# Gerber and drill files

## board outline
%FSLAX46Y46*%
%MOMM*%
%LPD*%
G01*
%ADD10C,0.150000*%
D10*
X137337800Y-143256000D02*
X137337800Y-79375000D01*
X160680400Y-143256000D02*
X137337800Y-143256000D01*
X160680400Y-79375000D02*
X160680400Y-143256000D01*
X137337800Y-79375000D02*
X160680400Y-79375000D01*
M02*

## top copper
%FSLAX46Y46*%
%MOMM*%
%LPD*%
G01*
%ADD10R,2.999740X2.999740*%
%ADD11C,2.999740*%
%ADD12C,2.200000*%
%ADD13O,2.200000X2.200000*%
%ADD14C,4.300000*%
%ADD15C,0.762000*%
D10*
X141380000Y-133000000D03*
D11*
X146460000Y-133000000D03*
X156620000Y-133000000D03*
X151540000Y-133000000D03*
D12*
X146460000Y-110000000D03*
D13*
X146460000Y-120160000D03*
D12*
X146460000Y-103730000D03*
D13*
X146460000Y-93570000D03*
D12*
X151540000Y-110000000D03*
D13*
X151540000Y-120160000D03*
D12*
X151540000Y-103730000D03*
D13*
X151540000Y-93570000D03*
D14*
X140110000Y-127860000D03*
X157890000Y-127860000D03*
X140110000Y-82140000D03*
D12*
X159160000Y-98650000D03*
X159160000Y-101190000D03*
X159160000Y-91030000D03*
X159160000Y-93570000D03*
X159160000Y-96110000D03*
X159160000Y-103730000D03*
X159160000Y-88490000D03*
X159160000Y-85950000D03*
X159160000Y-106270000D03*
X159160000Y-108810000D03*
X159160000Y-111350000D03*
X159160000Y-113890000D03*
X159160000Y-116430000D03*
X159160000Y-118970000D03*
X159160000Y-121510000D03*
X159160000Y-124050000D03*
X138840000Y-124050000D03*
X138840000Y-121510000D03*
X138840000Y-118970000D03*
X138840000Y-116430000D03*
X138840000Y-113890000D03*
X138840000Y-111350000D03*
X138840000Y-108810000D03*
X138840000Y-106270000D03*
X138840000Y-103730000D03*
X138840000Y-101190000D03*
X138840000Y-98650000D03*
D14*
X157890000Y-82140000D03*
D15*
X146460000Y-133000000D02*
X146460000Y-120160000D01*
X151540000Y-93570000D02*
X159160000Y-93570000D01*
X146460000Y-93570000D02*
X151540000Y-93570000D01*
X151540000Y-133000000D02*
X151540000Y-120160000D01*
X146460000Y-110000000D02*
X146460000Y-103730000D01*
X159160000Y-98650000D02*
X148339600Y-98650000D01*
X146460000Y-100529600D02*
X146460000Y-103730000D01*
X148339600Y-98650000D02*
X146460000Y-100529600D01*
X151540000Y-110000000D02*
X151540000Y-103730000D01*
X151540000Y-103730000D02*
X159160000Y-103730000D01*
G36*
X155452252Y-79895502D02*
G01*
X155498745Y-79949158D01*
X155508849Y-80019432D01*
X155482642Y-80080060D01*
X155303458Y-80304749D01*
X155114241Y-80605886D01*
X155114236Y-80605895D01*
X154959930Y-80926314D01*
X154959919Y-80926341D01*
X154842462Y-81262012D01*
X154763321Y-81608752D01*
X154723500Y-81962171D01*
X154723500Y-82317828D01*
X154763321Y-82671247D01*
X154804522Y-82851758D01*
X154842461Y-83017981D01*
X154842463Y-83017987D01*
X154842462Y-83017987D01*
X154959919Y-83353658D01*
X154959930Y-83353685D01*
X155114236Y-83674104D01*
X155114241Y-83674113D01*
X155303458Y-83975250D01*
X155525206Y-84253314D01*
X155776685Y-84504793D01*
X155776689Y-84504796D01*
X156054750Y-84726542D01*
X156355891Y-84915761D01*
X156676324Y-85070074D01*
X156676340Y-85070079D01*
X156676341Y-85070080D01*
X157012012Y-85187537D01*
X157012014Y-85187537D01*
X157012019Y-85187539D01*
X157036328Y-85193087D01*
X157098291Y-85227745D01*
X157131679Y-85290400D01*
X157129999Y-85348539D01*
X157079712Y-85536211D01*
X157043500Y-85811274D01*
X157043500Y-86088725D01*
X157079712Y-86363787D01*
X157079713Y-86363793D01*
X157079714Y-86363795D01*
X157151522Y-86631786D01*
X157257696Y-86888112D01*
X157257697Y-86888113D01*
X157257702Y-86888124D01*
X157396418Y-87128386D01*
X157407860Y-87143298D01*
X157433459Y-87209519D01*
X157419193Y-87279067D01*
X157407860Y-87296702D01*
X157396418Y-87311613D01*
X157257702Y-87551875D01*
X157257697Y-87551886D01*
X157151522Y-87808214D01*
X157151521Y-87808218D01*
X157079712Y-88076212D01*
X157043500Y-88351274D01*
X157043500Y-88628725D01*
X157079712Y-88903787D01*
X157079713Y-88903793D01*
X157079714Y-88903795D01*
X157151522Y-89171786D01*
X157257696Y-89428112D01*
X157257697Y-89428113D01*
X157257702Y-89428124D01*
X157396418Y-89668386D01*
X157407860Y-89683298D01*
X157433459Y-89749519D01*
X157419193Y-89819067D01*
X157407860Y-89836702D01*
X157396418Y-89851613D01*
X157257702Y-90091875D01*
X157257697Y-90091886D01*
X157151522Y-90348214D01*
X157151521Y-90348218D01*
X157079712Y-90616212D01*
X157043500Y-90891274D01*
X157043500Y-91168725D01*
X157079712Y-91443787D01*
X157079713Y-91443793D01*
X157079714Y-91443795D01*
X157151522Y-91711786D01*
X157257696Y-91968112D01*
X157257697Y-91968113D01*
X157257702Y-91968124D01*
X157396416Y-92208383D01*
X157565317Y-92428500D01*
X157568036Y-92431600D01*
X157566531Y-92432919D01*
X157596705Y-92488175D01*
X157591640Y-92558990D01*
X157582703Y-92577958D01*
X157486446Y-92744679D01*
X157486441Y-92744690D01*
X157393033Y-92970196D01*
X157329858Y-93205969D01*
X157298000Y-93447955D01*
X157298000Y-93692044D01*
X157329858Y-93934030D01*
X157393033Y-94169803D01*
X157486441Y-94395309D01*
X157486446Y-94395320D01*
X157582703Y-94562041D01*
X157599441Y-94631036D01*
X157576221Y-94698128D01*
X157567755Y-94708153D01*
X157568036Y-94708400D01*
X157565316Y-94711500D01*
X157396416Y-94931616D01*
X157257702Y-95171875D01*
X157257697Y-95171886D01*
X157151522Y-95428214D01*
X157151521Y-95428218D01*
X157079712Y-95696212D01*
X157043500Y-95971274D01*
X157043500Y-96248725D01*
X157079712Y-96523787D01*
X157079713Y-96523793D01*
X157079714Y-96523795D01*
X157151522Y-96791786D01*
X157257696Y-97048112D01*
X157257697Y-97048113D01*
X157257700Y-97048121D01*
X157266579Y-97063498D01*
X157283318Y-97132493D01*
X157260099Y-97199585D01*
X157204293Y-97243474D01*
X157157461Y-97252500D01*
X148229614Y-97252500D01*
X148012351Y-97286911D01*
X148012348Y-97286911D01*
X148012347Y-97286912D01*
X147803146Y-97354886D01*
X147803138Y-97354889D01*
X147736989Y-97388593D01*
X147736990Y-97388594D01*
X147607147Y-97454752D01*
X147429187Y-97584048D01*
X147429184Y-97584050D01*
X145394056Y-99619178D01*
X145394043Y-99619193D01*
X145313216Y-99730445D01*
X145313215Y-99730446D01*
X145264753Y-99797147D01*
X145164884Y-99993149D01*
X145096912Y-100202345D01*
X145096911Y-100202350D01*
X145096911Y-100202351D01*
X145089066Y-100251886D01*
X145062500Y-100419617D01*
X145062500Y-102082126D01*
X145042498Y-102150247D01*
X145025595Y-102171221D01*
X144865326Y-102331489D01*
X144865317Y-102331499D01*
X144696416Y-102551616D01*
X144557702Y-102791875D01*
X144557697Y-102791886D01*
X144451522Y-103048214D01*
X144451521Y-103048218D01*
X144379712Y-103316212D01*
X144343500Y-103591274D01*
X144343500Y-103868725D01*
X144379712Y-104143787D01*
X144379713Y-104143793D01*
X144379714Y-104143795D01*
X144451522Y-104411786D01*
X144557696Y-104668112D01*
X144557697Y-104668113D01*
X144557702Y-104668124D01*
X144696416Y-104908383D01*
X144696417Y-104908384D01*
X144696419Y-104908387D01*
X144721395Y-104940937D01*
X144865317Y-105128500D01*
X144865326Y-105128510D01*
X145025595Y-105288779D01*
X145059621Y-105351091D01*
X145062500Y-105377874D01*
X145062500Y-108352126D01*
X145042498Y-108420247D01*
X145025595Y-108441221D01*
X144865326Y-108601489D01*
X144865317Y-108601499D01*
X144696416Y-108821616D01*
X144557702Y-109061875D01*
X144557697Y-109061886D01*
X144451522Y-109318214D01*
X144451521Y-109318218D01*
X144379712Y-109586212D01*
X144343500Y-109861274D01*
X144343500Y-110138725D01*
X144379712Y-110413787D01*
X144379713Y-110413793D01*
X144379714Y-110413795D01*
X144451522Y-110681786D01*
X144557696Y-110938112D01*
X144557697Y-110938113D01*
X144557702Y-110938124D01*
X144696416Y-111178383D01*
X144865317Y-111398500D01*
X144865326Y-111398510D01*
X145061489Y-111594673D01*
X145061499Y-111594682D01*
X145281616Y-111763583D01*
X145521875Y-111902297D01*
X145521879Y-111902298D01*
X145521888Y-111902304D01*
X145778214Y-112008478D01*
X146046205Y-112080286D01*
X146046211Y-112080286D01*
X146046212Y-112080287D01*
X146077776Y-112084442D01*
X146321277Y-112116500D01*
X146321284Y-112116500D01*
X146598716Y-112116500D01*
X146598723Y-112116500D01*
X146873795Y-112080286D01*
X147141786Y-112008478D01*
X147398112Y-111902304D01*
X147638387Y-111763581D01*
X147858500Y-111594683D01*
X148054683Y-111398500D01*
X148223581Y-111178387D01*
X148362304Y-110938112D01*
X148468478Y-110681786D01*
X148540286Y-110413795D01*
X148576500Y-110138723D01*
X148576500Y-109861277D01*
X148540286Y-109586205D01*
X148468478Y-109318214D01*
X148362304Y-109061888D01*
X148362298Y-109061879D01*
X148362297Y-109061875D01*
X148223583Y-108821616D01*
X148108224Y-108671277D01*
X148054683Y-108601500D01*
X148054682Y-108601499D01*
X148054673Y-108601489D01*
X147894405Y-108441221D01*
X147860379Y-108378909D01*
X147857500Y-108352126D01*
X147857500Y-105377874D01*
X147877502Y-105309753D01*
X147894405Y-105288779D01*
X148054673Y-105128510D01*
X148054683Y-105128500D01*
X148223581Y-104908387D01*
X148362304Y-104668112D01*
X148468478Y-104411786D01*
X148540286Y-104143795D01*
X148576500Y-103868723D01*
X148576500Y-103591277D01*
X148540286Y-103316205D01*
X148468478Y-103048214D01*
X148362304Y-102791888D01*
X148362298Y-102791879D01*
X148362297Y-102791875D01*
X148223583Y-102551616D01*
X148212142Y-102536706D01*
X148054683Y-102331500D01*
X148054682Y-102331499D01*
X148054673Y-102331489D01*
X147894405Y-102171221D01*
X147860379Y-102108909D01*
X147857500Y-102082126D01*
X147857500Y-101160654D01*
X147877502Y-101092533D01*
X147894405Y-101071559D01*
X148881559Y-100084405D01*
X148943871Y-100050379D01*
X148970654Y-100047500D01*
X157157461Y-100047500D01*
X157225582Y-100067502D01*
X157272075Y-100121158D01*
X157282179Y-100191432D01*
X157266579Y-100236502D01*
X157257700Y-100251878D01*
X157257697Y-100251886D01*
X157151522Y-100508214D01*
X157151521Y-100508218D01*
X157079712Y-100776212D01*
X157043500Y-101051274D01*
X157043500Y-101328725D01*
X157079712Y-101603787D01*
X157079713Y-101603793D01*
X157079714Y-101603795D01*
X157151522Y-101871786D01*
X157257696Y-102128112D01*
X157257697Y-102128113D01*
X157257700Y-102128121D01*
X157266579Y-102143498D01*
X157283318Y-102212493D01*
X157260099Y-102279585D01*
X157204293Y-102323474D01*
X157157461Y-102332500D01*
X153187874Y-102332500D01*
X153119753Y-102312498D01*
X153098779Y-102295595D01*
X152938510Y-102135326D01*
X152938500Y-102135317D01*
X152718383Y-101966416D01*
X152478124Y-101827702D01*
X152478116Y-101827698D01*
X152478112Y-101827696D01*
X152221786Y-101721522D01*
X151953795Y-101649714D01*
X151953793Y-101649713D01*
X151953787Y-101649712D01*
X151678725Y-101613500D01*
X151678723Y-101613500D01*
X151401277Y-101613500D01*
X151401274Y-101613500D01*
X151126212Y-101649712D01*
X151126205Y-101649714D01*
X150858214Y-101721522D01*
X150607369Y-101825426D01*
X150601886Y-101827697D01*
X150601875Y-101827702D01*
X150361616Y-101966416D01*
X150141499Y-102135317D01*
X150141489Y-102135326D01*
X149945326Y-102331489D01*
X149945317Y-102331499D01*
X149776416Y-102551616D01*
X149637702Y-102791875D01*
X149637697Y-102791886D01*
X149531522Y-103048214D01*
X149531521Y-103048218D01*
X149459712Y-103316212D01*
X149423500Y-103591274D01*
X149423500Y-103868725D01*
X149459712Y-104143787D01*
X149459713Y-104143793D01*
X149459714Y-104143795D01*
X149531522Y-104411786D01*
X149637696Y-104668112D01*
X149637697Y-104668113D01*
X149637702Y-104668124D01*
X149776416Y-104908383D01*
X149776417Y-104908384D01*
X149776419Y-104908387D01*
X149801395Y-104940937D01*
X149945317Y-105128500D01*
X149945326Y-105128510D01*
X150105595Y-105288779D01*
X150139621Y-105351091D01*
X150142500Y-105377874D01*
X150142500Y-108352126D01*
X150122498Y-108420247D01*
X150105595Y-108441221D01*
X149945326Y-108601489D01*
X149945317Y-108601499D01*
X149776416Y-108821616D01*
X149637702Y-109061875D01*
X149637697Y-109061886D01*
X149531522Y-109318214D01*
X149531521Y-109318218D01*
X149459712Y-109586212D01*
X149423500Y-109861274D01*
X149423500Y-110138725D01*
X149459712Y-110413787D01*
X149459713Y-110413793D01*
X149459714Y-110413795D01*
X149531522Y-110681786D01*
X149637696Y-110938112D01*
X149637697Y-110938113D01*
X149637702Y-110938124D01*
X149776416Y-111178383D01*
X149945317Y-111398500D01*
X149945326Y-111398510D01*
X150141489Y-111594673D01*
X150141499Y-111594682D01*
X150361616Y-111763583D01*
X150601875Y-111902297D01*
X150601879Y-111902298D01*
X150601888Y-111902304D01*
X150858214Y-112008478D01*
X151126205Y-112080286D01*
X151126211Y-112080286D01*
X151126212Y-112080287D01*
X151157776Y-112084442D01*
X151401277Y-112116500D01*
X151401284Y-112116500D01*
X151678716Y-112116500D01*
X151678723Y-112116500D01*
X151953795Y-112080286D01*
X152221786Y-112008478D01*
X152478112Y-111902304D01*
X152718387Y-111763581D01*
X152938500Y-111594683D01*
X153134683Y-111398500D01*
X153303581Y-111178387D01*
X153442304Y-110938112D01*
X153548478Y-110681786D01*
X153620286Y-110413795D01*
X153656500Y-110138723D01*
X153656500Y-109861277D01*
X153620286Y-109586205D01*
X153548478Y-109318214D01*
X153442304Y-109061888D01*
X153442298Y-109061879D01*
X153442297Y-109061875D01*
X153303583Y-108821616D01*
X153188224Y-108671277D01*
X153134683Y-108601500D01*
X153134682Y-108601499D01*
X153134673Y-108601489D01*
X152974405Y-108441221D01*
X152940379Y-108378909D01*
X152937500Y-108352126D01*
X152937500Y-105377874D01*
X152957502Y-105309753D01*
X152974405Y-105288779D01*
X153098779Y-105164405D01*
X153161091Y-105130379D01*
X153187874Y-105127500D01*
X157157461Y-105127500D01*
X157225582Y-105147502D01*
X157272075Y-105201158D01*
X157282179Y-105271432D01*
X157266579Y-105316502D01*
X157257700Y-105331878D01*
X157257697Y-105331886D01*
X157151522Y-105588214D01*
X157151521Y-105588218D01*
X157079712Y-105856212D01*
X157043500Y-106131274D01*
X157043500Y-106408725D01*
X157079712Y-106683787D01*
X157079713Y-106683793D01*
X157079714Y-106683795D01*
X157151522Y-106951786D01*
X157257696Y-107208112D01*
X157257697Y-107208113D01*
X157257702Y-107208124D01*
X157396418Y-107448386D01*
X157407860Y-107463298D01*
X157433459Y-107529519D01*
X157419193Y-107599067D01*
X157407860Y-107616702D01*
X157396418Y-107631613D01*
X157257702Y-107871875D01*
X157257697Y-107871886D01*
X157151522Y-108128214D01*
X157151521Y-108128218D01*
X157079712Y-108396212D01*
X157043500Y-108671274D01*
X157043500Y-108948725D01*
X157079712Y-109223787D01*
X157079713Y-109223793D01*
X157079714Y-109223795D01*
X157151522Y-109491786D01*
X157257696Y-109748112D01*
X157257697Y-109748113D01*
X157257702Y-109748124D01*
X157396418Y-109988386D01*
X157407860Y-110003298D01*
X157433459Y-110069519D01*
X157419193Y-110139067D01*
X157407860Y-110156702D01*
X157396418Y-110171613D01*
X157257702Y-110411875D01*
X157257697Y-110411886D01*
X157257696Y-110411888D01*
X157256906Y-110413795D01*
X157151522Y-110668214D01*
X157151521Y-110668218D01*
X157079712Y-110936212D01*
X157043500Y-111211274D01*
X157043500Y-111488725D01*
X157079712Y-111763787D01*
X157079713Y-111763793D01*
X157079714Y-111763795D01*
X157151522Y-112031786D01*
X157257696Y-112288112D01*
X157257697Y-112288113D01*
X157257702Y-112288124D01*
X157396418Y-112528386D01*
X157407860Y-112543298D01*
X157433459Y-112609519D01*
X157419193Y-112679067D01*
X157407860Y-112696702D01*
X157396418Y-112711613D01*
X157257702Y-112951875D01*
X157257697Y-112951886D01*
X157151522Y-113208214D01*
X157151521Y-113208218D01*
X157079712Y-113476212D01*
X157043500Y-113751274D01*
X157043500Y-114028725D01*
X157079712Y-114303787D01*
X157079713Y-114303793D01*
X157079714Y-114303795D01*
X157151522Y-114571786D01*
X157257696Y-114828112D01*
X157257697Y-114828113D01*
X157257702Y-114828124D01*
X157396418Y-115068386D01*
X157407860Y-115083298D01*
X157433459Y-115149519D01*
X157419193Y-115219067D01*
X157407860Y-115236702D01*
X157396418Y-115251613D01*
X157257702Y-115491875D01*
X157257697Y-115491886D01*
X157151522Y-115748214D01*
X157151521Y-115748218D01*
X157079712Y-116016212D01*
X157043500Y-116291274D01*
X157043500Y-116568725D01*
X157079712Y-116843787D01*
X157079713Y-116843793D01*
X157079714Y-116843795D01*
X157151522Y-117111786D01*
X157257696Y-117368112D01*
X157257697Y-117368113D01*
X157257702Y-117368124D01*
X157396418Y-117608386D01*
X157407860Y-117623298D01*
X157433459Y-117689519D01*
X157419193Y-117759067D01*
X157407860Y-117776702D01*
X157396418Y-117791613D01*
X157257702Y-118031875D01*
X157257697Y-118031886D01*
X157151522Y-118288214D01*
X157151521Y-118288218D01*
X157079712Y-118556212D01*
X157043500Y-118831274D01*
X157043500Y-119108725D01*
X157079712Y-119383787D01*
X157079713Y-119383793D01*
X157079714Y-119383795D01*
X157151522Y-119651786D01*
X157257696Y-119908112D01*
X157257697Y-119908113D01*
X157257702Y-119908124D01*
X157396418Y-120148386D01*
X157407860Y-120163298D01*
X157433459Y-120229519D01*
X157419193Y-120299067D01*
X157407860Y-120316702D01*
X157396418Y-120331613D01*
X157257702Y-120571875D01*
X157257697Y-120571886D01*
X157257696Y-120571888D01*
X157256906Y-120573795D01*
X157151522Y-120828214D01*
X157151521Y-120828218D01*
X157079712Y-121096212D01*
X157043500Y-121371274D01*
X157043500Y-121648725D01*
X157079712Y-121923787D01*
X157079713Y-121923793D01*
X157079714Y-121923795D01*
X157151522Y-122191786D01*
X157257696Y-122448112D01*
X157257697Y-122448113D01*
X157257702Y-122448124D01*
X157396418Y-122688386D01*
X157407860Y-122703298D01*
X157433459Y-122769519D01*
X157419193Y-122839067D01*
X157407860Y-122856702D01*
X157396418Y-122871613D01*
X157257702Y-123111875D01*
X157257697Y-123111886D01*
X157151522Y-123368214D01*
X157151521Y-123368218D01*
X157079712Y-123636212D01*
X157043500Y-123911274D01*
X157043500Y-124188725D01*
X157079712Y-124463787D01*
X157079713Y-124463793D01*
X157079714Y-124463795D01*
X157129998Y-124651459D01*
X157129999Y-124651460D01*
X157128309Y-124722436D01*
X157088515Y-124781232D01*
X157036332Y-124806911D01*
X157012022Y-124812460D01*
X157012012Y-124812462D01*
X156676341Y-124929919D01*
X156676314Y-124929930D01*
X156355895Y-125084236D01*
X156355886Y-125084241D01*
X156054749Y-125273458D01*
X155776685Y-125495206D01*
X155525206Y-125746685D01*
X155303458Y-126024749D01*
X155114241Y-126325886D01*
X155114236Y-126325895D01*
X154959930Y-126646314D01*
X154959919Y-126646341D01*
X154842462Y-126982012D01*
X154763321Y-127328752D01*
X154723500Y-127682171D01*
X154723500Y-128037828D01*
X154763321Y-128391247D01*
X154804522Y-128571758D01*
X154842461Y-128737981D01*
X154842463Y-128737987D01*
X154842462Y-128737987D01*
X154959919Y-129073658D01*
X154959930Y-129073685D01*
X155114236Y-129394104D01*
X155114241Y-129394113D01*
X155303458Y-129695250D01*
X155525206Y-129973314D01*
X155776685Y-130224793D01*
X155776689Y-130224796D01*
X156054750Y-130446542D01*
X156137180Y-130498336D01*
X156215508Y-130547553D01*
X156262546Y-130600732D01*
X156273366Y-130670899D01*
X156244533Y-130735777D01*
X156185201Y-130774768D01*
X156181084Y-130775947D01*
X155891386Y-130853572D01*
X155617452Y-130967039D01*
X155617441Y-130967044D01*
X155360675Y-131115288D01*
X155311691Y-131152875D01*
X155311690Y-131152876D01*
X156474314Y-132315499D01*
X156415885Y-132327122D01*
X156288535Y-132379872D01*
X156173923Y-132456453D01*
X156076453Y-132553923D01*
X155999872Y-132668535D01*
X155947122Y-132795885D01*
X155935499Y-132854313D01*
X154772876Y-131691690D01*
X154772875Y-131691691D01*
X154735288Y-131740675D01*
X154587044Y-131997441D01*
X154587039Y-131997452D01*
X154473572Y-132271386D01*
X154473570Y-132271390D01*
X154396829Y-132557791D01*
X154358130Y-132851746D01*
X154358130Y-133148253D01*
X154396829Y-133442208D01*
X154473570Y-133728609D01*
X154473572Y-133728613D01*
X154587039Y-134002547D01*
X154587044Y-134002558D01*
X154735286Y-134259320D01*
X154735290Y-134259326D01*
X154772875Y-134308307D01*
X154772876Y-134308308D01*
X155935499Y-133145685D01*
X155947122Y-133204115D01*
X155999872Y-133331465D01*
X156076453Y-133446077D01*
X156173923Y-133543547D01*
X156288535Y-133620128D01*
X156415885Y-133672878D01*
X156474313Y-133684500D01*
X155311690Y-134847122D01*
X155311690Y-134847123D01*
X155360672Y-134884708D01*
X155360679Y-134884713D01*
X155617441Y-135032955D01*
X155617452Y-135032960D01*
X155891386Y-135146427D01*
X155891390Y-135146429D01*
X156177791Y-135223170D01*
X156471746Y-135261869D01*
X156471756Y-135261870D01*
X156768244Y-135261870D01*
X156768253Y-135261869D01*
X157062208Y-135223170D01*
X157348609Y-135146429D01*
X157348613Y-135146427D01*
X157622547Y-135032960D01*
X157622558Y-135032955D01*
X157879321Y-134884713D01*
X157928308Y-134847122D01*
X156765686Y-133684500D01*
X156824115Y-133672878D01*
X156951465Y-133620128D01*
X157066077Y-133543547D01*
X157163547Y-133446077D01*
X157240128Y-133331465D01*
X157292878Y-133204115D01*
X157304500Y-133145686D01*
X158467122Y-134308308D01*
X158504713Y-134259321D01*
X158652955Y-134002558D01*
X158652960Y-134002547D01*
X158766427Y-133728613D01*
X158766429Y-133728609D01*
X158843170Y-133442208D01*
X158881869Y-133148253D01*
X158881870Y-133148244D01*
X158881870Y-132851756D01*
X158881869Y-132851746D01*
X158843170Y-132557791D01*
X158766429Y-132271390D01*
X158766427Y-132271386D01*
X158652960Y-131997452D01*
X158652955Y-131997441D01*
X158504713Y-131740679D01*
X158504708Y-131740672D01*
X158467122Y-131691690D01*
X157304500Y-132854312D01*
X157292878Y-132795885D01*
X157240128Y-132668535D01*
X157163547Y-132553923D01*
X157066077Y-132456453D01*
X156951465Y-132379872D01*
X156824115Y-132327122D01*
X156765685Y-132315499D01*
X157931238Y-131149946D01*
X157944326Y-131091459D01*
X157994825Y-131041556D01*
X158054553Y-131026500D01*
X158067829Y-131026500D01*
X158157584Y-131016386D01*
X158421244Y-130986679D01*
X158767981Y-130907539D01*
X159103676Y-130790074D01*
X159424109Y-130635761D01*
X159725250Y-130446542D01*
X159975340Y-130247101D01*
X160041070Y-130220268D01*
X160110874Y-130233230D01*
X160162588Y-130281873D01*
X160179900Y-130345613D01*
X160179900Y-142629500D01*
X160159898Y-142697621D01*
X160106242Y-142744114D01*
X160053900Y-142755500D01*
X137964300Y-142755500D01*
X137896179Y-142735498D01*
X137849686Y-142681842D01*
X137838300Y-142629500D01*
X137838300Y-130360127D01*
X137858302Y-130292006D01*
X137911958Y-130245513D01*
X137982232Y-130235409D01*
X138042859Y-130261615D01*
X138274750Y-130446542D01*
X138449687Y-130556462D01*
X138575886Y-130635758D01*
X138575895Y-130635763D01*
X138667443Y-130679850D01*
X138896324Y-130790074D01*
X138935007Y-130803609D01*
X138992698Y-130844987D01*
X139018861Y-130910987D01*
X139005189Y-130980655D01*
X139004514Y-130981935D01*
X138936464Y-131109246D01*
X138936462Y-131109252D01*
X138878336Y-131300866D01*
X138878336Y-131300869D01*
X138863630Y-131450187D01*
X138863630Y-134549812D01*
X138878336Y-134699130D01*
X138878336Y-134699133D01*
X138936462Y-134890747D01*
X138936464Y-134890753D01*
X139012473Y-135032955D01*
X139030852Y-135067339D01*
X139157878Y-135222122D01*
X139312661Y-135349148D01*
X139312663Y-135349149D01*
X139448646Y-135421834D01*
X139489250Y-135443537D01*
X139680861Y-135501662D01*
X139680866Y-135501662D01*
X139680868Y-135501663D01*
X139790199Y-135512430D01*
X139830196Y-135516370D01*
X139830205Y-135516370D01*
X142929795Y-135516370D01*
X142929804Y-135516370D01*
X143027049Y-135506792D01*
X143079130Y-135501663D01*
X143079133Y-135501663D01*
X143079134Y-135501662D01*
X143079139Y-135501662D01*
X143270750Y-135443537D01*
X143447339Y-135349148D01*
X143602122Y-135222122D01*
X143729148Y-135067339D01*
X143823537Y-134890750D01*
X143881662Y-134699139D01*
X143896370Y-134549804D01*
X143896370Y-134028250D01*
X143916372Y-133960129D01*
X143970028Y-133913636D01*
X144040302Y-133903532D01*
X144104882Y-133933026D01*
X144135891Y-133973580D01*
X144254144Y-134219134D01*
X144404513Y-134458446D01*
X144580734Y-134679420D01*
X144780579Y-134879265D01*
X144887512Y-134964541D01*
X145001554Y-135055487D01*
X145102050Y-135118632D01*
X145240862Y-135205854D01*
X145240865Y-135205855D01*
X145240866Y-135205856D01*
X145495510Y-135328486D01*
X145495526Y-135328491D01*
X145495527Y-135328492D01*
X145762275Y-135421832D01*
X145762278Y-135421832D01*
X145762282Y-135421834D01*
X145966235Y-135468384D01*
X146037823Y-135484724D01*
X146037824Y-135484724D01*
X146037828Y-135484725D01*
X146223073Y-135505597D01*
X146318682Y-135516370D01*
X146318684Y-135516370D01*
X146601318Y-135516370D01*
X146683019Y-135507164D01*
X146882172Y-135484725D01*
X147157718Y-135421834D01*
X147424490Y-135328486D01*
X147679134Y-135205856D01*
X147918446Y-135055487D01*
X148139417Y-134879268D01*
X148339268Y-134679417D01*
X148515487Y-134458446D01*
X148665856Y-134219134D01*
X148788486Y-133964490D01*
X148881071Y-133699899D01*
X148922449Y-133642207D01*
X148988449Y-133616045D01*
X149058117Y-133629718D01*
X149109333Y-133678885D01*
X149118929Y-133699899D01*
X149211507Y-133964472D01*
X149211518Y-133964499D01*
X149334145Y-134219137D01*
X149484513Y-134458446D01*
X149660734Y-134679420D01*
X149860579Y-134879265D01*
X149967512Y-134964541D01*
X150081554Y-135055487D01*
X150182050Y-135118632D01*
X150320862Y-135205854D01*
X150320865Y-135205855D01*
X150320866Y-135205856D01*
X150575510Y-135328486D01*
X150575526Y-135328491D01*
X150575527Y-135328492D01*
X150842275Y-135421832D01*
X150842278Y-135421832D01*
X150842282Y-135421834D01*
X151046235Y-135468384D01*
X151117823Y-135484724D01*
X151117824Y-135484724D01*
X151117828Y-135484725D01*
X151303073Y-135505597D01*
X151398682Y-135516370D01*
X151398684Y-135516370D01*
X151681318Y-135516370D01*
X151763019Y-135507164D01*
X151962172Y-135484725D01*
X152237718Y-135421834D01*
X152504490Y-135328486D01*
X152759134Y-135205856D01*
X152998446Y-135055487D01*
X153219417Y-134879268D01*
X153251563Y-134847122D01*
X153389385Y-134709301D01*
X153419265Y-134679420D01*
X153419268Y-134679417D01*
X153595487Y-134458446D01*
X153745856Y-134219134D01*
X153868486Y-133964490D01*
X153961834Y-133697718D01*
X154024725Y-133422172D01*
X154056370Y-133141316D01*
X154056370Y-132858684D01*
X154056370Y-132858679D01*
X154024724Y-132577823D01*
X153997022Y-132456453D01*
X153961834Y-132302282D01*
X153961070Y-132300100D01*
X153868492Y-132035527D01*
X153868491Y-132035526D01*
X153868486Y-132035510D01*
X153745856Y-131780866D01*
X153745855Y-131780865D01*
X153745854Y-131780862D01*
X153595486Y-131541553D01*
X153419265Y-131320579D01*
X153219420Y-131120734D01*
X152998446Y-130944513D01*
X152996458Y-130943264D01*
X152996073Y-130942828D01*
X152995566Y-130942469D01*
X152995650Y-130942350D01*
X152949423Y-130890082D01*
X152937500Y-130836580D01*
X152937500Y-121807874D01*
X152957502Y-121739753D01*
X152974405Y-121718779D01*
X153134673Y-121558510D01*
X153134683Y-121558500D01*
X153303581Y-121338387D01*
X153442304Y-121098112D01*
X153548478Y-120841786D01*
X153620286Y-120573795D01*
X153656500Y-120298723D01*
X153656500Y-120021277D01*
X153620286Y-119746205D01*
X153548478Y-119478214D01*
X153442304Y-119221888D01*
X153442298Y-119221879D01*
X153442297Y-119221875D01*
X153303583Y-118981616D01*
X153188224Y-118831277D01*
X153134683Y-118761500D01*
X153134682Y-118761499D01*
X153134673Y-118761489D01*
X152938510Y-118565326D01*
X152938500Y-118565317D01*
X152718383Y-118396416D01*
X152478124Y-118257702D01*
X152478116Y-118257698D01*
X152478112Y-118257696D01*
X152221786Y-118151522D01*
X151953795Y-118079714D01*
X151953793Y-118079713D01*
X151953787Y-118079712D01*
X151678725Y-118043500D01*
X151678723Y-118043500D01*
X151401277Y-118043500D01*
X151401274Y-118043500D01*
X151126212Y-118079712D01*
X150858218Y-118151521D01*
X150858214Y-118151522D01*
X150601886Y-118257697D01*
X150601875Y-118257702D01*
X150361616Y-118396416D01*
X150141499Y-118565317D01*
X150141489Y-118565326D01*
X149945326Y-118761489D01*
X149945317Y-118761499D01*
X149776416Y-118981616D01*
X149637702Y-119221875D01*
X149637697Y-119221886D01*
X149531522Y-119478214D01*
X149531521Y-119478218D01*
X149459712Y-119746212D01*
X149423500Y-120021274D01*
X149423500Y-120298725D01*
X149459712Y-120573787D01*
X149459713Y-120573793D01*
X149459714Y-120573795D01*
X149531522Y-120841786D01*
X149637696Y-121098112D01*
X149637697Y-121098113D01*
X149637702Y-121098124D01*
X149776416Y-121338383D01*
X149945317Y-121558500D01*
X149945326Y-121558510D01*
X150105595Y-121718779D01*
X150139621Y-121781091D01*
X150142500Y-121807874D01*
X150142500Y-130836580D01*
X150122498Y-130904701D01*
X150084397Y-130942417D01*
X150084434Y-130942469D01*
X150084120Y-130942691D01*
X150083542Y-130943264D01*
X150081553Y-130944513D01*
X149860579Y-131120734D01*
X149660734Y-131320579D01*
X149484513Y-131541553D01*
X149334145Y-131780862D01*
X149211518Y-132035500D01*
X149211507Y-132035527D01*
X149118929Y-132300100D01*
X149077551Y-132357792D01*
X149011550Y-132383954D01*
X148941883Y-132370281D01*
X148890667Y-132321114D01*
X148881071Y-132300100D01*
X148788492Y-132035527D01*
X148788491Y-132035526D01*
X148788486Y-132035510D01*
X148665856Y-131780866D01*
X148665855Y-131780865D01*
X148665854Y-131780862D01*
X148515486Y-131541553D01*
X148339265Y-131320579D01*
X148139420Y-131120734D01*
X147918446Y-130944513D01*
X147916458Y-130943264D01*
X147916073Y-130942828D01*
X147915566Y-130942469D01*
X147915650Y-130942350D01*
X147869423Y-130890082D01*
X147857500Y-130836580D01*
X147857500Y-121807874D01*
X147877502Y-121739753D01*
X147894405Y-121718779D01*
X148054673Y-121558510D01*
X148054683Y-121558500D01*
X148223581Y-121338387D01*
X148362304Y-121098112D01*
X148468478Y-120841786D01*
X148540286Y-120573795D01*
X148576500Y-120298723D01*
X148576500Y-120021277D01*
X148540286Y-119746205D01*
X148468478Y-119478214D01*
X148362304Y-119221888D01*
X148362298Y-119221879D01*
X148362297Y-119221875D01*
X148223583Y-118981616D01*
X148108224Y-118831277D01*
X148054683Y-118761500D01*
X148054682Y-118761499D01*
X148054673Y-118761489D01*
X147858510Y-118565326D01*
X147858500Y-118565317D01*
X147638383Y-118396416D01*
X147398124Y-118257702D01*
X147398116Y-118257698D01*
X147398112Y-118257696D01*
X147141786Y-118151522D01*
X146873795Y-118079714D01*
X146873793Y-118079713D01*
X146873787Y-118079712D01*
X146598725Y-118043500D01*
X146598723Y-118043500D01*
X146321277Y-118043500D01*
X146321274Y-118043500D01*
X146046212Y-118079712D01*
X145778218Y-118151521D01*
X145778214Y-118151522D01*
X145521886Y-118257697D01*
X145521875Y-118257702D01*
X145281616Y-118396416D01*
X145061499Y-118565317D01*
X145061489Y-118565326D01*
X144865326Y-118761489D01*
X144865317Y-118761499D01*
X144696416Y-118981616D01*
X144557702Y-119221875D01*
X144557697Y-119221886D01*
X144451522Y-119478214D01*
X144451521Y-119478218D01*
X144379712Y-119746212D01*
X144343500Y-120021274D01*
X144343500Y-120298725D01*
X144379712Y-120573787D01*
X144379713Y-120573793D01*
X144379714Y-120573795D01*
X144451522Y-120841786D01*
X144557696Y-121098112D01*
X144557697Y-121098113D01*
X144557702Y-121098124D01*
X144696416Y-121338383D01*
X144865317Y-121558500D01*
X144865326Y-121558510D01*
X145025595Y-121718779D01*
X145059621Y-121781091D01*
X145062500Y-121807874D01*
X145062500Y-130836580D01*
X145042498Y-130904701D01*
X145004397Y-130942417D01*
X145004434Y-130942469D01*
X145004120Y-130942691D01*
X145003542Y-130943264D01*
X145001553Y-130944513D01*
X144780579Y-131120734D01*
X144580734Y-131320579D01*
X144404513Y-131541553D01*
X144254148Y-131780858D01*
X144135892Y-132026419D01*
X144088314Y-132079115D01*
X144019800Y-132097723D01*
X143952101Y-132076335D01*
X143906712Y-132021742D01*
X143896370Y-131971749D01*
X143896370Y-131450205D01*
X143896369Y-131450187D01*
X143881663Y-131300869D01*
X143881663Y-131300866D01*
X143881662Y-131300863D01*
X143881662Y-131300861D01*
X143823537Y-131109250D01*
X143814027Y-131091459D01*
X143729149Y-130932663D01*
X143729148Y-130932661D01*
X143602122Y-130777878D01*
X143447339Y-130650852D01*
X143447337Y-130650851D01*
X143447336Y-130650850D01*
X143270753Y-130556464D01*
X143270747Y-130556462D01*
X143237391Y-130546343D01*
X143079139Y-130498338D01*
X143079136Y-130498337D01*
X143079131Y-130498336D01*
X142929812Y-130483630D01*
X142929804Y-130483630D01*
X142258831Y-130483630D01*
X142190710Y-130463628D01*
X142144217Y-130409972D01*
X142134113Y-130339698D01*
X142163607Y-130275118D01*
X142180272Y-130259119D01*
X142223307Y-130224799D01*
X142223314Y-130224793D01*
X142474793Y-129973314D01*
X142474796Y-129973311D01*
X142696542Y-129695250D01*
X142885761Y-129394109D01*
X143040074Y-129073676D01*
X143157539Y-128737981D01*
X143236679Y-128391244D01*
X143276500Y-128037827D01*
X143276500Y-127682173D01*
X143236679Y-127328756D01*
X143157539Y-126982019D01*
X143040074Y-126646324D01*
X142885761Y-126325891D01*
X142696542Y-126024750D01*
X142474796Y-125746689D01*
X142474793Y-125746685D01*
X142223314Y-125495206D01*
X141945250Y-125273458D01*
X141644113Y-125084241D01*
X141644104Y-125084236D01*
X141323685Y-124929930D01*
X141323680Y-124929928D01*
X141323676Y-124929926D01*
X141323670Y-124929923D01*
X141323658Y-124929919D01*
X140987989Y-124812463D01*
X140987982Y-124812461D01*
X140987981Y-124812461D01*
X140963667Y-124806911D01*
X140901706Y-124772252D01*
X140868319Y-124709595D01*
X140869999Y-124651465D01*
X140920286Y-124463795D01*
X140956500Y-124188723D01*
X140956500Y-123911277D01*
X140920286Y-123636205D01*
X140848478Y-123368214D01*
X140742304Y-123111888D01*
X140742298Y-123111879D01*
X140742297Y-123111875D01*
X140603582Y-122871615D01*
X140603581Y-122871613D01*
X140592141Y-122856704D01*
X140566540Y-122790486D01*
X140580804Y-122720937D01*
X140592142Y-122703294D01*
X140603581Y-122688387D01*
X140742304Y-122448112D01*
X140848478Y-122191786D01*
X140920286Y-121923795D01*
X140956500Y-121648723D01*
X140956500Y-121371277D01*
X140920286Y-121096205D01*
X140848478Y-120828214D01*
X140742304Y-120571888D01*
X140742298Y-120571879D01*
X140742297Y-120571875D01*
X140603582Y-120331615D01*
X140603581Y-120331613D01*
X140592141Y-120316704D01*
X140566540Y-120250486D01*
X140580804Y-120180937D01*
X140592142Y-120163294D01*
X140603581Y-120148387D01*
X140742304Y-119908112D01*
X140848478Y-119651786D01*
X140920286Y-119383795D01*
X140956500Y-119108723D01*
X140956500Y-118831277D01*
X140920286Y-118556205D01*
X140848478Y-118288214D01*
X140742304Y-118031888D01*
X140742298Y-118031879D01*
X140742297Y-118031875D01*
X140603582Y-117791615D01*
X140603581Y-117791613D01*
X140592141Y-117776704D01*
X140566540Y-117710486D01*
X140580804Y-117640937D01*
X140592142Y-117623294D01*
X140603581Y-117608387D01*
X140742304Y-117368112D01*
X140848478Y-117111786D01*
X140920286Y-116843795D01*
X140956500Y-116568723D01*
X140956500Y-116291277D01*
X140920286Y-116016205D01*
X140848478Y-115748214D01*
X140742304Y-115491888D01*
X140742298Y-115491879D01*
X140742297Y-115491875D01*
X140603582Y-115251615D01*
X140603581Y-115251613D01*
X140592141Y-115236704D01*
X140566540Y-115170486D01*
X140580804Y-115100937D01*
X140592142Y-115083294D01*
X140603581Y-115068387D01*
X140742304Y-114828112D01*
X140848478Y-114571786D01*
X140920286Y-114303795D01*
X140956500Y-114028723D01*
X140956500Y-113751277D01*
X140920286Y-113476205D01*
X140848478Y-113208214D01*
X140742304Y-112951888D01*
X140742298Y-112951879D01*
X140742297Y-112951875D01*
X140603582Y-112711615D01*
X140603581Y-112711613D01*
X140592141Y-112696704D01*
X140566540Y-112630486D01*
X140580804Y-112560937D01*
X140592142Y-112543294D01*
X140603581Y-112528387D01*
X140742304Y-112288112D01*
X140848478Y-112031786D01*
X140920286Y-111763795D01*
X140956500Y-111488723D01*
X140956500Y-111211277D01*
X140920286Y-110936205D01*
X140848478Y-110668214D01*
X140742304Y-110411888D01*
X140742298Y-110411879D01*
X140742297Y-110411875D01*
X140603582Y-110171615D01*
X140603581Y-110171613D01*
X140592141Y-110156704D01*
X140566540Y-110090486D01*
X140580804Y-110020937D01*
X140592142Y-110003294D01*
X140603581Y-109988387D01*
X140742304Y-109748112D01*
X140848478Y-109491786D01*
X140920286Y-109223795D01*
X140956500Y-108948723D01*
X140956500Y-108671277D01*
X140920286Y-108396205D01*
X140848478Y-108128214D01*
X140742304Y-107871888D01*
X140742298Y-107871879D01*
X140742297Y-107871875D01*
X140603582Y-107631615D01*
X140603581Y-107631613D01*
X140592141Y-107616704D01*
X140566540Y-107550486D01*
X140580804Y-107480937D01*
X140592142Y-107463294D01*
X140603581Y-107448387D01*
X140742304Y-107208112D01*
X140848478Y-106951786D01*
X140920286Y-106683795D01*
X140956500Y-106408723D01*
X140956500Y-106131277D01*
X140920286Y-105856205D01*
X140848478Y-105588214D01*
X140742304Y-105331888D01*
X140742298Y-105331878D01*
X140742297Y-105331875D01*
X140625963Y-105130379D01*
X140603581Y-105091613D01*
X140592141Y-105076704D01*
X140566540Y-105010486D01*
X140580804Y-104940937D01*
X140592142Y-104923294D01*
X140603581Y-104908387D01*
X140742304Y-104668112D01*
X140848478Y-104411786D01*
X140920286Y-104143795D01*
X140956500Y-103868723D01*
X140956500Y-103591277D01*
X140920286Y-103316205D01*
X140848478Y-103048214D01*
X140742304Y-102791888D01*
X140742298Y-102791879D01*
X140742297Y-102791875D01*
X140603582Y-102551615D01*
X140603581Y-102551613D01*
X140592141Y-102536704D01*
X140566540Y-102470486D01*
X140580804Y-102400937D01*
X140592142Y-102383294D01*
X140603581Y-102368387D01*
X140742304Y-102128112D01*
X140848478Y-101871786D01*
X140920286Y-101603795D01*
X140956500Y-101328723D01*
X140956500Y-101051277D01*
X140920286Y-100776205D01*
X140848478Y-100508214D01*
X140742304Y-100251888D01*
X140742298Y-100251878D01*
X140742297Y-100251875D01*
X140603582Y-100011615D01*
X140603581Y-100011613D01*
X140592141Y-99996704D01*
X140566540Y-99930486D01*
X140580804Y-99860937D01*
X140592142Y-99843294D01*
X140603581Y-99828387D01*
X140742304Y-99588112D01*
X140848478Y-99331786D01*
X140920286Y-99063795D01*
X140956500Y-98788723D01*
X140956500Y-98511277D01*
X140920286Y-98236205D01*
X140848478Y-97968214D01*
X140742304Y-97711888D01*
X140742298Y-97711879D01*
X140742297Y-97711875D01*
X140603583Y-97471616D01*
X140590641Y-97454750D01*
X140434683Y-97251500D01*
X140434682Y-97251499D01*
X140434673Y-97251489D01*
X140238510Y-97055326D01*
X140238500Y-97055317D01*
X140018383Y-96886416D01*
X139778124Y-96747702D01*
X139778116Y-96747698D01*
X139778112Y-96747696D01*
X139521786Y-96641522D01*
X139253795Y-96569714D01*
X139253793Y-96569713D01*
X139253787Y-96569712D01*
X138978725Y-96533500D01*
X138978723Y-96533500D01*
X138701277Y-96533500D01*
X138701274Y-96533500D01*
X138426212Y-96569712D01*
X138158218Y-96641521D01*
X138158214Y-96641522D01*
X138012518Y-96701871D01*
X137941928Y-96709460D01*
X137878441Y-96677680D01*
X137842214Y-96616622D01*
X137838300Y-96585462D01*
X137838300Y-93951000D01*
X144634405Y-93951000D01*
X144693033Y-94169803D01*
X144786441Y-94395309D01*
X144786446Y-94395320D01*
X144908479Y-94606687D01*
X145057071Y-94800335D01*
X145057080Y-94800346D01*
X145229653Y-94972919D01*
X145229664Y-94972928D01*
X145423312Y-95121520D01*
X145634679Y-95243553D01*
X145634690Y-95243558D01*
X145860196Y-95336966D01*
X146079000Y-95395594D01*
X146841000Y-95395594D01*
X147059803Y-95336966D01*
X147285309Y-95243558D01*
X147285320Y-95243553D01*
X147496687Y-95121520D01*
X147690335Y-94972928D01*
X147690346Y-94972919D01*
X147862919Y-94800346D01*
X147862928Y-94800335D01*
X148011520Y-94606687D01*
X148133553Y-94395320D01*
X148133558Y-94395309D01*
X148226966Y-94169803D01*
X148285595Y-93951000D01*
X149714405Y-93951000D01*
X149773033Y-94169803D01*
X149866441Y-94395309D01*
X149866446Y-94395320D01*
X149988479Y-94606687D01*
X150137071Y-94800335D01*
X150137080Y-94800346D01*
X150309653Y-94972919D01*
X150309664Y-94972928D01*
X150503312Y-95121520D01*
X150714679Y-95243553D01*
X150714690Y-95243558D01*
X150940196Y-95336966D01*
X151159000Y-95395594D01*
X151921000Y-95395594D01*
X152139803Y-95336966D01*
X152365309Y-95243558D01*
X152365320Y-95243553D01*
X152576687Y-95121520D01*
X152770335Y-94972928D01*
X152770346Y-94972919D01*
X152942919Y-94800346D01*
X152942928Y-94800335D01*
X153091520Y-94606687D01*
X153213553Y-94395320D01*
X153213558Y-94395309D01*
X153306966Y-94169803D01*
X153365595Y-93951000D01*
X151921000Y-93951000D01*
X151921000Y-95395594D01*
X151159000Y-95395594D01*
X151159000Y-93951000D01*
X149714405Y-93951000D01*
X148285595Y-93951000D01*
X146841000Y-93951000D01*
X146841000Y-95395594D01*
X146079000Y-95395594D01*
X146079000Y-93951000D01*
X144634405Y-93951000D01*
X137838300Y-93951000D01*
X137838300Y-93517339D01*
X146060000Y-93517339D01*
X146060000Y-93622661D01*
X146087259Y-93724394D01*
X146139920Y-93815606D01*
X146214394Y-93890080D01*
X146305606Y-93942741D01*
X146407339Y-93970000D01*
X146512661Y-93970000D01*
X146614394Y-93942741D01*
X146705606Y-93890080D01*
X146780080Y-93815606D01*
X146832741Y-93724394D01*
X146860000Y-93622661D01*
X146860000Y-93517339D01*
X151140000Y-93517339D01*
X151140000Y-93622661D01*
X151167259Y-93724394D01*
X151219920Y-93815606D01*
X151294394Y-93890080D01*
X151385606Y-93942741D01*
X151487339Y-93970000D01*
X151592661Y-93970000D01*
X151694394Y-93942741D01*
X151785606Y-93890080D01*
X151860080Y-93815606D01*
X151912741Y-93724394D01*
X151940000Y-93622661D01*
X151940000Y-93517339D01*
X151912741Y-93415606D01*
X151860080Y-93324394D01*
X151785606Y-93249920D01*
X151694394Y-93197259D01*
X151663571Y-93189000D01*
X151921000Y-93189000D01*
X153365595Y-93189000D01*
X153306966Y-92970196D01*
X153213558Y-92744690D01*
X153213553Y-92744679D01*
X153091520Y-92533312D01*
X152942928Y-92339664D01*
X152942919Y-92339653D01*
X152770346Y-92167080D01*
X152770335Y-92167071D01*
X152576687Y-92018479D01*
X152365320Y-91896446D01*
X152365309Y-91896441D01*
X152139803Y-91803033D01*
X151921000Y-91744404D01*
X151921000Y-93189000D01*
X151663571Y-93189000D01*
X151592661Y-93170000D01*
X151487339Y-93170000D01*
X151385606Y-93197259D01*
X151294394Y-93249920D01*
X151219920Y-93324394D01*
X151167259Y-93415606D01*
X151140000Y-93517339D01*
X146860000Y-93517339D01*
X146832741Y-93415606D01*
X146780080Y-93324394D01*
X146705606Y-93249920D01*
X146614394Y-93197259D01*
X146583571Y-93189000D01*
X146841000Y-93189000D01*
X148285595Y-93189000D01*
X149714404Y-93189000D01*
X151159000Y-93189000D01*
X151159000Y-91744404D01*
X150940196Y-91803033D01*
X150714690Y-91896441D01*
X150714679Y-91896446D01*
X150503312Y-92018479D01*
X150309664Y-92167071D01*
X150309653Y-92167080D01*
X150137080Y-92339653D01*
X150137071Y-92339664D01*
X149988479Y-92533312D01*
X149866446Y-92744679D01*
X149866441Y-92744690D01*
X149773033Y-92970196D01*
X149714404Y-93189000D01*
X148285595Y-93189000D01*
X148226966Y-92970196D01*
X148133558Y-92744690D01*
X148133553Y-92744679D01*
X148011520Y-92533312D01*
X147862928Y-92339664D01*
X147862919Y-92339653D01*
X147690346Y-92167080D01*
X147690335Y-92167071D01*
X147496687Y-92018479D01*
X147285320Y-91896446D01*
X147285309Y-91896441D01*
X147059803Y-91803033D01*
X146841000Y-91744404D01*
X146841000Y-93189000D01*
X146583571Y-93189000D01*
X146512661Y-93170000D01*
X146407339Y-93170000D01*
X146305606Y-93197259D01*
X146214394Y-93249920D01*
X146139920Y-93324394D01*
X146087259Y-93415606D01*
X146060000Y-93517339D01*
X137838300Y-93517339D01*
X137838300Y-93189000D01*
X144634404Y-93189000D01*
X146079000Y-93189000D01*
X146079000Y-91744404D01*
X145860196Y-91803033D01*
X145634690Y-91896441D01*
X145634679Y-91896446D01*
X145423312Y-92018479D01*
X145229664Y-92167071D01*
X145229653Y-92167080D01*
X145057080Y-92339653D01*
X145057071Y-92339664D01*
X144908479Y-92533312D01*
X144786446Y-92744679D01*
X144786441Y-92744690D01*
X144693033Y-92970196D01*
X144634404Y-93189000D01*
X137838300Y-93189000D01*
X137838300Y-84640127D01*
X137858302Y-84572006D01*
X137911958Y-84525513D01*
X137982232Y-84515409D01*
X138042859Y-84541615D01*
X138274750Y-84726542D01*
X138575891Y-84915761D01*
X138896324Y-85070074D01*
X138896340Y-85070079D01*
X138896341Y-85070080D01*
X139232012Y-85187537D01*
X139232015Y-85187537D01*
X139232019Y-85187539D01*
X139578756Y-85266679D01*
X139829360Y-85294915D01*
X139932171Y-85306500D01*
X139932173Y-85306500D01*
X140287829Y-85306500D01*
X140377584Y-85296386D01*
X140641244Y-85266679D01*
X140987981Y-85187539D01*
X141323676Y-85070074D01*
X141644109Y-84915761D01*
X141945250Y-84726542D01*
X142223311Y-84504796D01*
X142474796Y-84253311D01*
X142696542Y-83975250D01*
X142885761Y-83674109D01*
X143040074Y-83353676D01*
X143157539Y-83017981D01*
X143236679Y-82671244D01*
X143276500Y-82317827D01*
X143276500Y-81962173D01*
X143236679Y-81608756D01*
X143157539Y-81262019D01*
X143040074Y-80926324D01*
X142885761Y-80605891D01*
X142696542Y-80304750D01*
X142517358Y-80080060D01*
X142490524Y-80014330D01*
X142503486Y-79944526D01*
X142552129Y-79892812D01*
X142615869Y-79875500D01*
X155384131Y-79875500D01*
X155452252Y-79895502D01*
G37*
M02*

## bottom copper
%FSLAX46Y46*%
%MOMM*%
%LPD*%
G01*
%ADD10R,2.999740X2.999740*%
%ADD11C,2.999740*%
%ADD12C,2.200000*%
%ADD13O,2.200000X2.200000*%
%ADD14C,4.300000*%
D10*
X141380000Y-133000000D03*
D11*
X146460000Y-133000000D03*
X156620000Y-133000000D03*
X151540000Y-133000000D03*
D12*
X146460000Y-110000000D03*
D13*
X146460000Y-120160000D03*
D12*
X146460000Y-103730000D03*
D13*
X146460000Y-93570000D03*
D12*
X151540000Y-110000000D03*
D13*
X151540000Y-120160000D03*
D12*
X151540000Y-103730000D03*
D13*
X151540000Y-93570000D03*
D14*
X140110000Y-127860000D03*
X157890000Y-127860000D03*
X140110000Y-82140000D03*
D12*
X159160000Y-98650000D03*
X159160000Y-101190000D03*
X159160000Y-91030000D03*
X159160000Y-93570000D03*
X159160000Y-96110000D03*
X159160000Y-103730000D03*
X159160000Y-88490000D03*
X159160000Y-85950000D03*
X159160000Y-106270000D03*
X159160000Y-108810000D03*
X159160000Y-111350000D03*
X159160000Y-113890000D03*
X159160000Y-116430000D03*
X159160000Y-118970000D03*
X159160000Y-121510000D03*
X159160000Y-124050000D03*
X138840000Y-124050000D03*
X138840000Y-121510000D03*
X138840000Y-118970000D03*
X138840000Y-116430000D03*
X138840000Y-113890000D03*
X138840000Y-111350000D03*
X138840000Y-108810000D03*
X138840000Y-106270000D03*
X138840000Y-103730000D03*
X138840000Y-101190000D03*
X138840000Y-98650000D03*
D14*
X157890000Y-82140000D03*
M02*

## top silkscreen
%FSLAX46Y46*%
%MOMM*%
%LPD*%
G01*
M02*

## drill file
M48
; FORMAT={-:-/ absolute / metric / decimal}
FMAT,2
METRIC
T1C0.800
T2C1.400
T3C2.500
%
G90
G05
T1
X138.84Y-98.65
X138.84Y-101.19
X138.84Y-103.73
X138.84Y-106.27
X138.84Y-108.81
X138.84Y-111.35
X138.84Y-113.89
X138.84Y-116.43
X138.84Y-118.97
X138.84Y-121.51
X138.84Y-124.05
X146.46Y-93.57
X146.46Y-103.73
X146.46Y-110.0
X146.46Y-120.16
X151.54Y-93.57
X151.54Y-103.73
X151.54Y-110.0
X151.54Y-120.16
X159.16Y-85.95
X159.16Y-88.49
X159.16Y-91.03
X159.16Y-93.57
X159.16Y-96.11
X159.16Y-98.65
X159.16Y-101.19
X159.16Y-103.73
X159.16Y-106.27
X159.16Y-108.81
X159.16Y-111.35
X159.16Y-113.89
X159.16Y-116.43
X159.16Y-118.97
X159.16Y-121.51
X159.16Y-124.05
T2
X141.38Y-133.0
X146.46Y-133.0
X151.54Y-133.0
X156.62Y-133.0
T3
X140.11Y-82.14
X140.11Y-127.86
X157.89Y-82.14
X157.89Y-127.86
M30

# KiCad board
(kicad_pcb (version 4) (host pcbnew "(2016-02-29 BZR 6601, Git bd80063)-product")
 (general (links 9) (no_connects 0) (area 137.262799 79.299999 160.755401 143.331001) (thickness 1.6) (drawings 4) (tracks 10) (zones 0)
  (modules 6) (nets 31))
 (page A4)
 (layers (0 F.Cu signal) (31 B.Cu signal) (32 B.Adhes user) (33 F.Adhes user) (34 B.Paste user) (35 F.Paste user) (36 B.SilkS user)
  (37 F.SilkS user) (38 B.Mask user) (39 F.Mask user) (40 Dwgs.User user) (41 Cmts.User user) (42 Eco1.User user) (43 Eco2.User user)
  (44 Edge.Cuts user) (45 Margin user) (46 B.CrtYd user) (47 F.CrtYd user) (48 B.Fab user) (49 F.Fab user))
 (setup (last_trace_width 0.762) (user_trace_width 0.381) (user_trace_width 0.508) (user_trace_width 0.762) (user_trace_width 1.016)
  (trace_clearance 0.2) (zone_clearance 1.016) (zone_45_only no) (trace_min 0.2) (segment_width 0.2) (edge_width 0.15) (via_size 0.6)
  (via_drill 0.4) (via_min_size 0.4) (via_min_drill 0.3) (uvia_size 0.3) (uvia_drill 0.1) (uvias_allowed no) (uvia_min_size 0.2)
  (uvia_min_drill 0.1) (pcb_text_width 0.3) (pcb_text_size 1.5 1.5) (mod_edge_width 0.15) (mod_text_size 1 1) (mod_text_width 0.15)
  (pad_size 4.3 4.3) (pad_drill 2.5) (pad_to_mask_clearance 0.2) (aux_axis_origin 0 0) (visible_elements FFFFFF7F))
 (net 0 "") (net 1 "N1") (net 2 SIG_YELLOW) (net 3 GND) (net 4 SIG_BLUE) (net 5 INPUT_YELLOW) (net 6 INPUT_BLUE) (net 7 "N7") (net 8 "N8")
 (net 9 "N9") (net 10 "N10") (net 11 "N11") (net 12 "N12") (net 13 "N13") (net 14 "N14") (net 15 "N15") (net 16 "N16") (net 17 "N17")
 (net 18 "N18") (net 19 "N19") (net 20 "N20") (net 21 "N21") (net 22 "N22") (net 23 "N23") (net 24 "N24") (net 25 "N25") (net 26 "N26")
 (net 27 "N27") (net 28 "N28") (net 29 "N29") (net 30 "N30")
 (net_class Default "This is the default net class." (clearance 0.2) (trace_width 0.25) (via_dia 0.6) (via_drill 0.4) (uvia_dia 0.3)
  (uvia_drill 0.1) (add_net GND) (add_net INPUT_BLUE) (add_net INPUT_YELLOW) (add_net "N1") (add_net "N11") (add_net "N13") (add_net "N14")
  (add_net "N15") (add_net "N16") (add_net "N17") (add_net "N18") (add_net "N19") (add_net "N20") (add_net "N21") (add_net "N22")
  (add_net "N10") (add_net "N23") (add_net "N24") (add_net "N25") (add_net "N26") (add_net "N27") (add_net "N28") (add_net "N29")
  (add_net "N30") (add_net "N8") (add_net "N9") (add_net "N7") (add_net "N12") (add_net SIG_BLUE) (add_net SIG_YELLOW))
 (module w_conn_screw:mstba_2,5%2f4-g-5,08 (layer B.Cu) (at 149 133)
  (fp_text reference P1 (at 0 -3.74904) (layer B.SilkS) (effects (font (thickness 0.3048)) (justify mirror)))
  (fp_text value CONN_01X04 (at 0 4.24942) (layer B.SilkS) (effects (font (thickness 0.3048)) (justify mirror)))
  (pad 1 thru_hole rect (at -7.62 0) (size 2.99974 2.99974) (drill 1.39954) (layers *.Cu *.Mask B.SilkS) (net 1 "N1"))
  (pad 2 thru_hole circle (at -2.54 0) (size 2.99974 2.99974) (drill 1.39954) (layers *.Cu *.Mask B.SilkS) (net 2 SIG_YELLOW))
  (pad 4 thru_hole circle (at 7.62 0) (size 2.99974 2.99974) (drill 1.39954) (layers *.Cu *.Mask B.SilkS) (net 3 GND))
  (pad 3 thru_hole circle (at 2.54 0) (size 2.99974 2.99974) (drill 1.39954) (layers *.Cu *.Mask B.SilkS) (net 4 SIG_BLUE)))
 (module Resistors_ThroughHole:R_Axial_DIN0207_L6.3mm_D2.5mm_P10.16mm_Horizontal (layer B.Cu) (at 146.46 110 270)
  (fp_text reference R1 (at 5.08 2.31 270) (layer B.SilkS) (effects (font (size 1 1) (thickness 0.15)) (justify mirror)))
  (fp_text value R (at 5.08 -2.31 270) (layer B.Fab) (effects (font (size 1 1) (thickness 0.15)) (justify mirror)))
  (pad 1 thru_hole circle (at 0 0 270) (size 2.2 2.2) (drill 0.8) (layers *.Cu *.Mask) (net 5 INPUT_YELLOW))
  (pad 2 thru_hole oval (at 10.16 0 270) (size 2.2 2.2) (drill 0.8) (layers *.Cu *.Mask) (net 2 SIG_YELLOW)))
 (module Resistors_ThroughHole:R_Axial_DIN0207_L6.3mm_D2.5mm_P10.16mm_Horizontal (layer B.Cu) (at 146.46 103.73 90)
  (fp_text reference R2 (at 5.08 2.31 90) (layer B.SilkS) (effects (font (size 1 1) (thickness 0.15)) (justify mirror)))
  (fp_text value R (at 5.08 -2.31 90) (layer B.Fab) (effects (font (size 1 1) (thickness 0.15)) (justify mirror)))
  (pad 1 thru_hole circle (at 0 0 90) (size 2.2 2.2) (drill 0.8) (layers *.Cu *.Mask) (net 5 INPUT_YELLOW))
  (pad 2 thru_hole oval (at 10.16 0 90) (size 2.2 2.2) (drill 0.8) (layers *.Cu *.Mask) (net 3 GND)))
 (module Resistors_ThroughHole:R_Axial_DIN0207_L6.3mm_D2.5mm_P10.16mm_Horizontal (layer B.Cu) (at 151.54 110 270)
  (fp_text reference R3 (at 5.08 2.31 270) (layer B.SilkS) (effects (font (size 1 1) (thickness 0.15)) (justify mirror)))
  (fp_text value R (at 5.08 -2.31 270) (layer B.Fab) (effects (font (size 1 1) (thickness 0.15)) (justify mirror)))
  (pad 1 thru_hole circle (at 0 0 270) (size 2.2 2.2) (drill 0.8) (layers *.Cu *.Mask) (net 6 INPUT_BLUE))
  (pad 2 thru_hole oval (at 10.16 0 270) (size 2.2 2.2) (drill 0.8) (layers *.Cu *.Mask) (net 4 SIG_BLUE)))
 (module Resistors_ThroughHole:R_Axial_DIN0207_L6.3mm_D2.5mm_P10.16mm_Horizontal (layer B.Cu) (at 151.54 103.73 90)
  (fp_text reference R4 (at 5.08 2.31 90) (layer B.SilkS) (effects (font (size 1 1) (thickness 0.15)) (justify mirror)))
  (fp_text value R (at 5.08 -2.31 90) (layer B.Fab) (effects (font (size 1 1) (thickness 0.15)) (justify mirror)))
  (pad 1 thru_hole circle (at 0 0 90) (size 2.2 2.2) (drill 0.8) (layers *.Cu *.Mask) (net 6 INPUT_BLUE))
  (pad 2 thru_hole oval (at 10.16 0 90) (size 2.2 2.2) (drill 0.8) (layers *.Cu *.Mask) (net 3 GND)))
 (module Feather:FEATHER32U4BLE (layer B.Cu) (at 149 105 180)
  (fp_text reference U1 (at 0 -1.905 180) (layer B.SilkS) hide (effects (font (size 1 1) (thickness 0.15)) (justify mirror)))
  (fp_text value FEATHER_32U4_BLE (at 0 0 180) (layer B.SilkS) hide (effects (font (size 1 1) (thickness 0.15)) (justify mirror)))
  (pad "" thru_hole circle (at 8.89 -22.86 180) (size 4.3 4.3) (drill 2.5) (layers *.Cu *.Mask B.SilkS))
  (pad "" thru_hole circle (at -8.89 -22.86 180) (size 4.3 4.3) (drill 2.5) (layers *.Cu *.Mask B.SilkS))
  (pad "" thru_hole circle (at 8.89 22.86 180) (size 4.3 4.3) (drill 2.5) (layers *.Cu *.Mask B.SilkS))
  (pad 6 thru_hole circle (at -10.16 6.35 180) (size 2.2 2.2) (drill 0.8) (layers *.Cu *.Mask B.SilkS) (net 5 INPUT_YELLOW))
  (pad 7 thru_hole circle (at -10.16 3.81 180) (size 2.2 2.2) (drill 0.8) (layers *.Cu *.Mask B.SilkS) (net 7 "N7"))
  (pad 3 thru_hole circle (at -10.16 13.97 180) (size 2.2 2.2) (drill 0.8) (layers *.Cu *.Mask B.SilkS) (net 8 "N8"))
  (pad 4 thru_hole circle (at -10.16 11.43 180) (size 2.2 2.2) (drill 0.8) (layers *.Cu *.Mask B.SilkS) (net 3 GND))
  (pad 5 thru_hole circle (at -10.16 8.89 180) (size 2.2 2.2) (drill 0.8) (layers *.Cu *.Mask B.SilkS) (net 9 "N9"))
  (pad 8 thru_hole circle (at -10.16 1.27 180) (size 2.2 2.2) (drill 0.8) (layers *.Cu *.Mask B.SilkS) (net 6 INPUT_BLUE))
  (pad 2 thru_hole circle (at -10.16 16.51 180) (size 2.2 2.2) (drill 0.8) (layers *.Cu *.Mask B.SilkS) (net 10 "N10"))
  (pad 1 thru_hole circle (at -10.16 19.05 180) (size 2.2 2.2) (drill 0.8) (layers *.Cu *.Mask B.SilkS) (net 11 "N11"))
  (pad 9 thru_hole circle (at -10.16 -1.27 180) (size 2.2 2.2) (drill 0.8) (layers *.Cu *.Mask B.SilkS) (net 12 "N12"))
  (pad 10 thru_hole circle (at -10.16 -3.81 180) (size 2.2 2.2) (drill 0.8) (layers *.Cu *.Mask B.SilkS) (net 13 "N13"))
  (pad 11 thru_hole circle (at -10.16 -6.35 180) (size 2.2 2.2) (drill 0.8) (layers *.Cu *.Mask B.SilkS) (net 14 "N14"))
  (pad 12 thru_hole circle (at -10.16 -8.89 180) (size 2.2 2.2) (drill 0.8) (layers *.Cu *.Mask B.SilkS) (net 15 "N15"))
  (pad 13 thru_hole circle (at -10.16 -11.43 180) (size 2.2 2.2) (drill 0.8) (layers *.Cu *.Mask B.SilkS) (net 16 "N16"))
  (pad 14 thru_hole circle (at -10.16 -13.97 180) (size 2.2 2.2) (drill 0.8) (layers *.Cu *.Mask B.SilkS) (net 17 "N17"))
  (pad 15 thru_hole circle (at -10.16 -16.51 180) (size 2.2 2.2) (drill 0.8) (layers *.Cu *.Mask B.SilkS) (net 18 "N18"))
  (pad 16 thru_hole circle (at -10.16 -19.05 180) (size 2.2 2.2) (drill 0.8) (layers *.Cu *.Mask B.SilkS) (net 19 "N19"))
  (pad 17 thru_hole circle (at 10.16 -19.05 180) (size 2.2 2.2) (drill 0.8) (layers *.Cu *.Mask B.SilkS) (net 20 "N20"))
  (pad 18 thru_hole circle (at 10.16 -16.51 180) (size 2.2 2.2) (drill 0.8) (layers *.Cu *.Mask B.SilkS) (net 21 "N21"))
  (pad 19 thru_hole circle (at 10.16 -13.97 180) (size 2.2 2.2) (drill 0.8) (layers *.Cu *.Mask B.SilkS) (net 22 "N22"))
  (pad 20 thru_hole circle (at 10.16 -11.43 180) (size 2.2 2.2) (drill 0.8) (layers *.Cu *.Mask B.SilkS) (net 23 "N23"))
  (pad 21 thru_hole circle (at 10.16 -8.89 180) (size 2.2 2.2) (drill 0.8) (layers *.Cu *.Mask B.SilkS) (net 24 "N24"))
  (pad 22 thru_hole circle (at 10.16 -6.35 180) (size 2.2 2.2) (drill 0.8) (layers *.Cu *.Mask B.SilkS) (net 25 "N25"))
  (pad 23 thru_hole circle (at 10.16 -3.81 180) (size 2.2 2.2) (drill 0.8) (layers *.Cu *.Mask B.SilkS) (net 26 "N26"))
  (pad 24 thru_hole circle (at 10.16 -1.27 180) (size 2.2 2.2) (drill 0.8) (layers *.Cu *.Mask B.SilkS) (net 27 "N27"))
  (pad 25 thru_hole circle (at 10.16 1.27 180) (size 2.2 2.2) (drill 0.8) (layers *.Cu *.Mask B.SilkS) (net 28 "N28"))
  (pad 26 thru_hole circle (at 10.16 3.81 180) (size 2.2 2.2) (drill 0.8) (layers *.Cu *.Mask B.SilkS) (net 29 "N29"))
  (pad 27 thru_hole circle (at 10.16 6.35 180) (size 2.2 2.2) (drill 0.8) (layers *.Cu *.Mask B.SilkS) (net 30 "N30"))
  (pad "" thru_hole circle (at -8.89 22.86 180) (size 4.3 4.3) (drill 2.5) (layers *.Cu *.Mask B.SilkS)))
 (gr_line (start 137.3378 143.256) (end 137.3378 79.375) (angle 90) (layer Edge.Cuts) (width 0.15))
 (gr_line (start 160.6804 143.256) (end 137.3378 143.256) (angle 90) (layer Edge.Cuts) (width 0.15))
 (gr_line (start 160.6804 79.375) (end 160.6804 143.256) (angle 90) (layer Edge.Cuts) (width 0.15))
 (gr_line (start 137.3378 79.375) (end 160.6804 79.375) (angle 90) (layer Edge.Cuts) (width 0.15))
 (segment (start 146.46 133) (end 146.46 120.16) (width 0.762) (layer F.Cu) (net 2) (status C00000))
 (segment (start 151.54 93.57) (end 159.16 93.57) (width 0.762) (layer F.Cu) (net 3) (status C00000))
 (segment (start 146.46 93.57) (end 151.54 93.57) (width 0.762) (layer F.Cu) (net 3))
 (segment (start 151.54 133) (end 151.54 120.16) (width 0.762) (layer F.Cu) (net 4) (status C00000))
 (segment (start 146.46 110) (end 146.46 103.73) (width 0.762) (layer F.Cu) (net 5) (status C00000))
 (segment (start 159.16 98.65) (end 148.3396 98.65) (width 0.762) (layer F.Cu) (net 5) (status 400000))
 (segment (start 146.46 100.5296) (end 146.46 103.73) (width 0.762) (layer F.Cu) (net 5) (status 800000))
 (segment (start 148.3396 98.65) (end 146.46 100.5296) (width 0.762) (layer F.Cu) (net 5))
 (segment (start 151.54 110) (end 151.54 103.73) (width 0.762) (layer F.Cu) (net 6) (status C00000))
 (segment (start 151.54 103.73) (end 159.16 103.73) (width 0.762) (layer F.Cu) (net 6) (status C00000))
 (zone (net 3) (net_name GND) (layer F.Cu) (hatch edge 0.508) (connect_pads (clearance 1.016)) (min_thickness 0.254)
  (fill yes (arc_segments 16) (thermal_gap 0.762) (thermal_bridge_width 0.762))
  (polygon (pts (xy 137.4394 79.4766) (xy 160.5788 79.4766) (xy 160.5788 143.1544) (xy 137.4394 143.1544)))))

